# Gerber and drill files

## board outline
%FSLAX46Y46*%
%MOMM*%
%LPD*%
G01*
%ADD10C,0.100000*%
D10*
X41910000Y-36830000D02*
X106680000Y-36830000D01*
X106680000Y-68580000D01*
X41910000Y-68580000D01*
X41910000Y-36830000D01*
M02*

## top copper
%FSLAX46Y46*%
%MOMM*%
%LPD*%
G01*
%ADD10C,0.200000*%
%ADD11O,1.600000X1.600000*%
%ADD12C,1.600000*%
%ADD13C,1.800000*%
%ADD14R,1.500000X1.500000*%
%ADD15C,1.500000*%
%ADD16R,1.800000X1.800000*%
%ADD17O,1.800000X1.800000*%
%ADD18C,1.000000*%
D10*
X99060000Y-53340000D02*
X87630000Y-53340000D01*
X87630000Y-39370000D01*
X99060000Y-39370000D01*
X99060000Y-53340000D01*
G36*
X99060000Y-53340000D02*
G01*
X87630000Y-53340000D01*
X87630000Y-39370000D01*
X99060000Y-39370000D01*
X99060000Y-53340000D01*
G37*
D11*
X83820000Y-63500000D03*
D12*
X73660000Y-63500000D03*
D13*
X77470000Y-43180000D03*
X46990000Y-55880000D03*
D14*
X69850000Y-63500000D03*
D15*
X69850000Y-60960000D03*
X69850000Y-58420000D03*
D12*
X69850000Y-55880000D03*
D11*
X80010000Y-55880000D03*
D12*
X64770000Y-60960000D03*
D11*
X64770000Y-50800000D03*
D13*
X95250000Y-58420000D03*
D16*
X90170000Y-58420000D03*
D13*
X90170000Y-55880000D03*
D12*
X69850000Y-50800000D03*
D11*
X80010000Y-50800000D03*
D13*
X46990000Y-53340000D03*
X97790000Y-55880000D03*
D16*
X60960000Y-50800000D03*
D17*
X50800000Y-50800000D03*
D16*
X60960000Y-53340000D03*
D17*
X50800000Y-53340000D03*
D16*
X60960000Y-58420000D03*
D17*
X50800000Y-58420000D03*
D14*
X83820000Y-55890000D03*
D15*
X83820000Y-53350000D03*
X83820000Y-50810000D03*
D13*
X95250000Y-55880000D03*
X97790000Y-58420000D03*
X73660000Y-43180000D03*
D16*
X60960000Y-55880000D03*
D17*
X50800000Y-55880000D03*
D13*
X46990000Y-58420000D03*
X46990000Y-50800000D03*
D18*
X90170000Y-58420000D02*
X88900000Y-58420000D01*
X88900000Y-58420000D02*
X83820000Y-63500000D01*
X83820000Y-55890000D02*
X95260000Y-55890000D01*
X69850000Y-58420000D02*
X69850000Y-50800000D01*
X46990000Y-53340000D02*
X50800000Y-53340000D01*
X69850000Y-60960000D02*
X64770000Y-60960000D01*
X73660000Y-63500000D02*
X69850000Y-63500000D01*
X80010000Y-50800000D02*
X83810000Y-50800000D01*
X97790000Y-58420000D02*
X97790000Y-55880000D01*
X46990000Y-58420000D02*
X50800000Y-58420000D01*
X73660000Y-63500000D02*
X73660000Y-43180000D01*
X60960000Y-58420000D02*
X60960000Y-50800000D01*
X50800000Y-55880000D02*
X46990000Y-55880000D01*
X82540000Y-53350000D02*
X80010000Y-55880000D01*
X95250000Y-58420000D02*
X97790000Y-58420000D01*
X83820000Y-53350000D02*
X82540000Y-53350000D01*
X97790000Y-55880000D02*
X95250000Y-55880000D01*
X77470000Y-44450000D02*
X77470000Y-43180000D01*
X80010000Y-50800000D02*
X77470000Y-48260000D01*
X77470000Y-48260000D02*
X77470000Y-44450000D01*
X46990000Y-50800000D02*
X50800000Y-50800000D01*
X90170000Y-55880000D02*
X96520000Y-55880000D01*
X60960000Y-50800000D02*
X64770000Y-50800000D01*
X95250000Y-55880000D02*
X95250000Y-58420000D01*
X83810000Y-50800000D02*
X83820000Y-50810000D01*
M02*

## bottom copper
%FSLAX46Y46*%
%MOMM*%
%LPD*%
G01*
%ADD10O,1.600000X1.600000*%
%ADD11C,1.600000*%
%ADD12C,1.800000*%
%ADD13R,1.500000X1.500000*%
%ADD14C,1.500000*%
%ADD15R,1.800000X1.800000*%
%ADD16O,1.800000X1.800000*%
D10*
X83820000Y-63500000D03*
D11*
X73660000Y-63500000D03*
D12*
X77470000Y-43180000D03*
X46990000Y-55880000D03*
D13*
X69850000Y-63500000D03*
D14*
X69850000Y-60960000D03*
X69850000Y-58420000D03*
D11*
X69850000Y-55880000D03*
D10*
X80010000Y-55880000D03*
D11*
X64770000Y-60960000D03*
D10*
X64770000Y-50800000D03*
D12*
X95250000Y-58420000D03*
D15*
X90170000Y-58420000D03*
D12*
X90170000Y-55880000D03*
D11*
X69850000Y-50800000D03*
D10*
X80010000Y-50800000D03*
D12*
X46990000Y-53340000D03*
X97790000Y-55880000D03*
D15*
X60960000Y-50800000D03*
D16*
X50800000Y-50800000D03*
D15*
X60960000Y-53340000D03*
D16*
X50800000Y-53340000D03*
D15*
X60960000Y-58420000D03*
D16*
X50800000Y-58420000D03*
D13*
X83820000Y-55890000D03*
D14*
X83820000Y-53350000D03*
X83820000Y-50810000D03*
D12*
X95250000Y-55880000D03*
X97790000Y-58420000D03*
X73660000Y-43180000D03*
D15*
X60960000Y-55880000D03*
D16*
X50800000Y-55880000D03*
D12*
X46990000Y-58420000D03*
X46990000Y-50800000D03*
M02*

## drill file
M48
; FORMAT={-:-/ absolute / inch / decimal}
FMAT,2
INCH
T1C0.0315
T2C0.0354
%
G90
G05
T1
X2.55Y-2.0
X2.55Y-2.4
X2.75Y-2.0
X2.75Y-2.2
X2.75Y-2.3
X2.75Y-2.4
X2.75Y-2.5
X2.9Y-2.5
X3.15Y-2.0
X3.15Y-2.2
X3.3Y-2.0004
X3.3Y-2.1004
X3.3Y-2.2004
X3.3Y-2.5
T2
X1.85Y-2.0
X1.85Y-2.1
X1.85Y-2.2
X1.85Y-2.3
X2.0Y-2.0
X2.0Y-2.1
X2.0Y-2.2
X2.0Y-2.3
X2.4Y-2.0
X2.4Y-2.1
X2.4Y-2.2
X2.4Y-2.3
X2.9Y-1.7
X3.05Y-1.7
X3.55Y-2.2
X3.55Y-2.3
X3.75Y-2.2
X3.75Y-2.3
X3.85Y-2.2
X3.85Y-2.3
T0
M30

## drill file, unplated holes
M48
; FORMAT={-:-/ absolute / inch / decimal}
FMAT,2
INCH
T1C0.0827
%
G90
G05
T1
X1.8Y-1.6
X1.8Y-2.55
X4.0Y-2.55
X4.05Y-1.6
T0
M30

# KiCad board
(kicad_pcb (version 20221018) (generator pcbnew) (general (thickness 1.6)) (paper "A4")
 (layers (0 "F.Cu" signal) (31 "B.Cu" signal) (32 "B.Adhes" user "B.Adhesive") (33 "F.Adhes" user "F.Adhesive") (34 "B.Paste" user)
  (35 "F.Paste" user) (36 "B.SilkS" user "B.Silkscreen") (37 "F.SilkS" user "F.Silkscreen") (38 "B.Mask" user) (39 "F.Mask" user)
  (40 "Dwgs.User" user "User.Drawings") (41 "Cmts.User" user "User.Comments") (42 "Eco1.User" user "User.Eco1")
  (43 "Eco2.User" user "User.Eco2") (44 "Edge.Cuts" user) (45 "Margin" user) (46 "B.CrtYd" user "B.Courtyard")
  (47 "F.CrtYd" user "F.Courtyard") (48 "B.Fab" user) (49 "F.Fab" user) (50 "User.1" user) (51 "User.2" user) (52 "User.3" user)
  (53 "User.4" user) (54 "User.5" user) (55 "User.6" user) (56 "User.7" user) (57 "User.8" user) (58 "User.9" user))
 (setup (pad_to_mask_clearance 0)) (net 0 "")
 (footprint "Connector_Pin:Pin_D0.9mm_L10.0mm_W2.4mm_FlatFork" (layer "F.Cu") (at 77.47 43.18)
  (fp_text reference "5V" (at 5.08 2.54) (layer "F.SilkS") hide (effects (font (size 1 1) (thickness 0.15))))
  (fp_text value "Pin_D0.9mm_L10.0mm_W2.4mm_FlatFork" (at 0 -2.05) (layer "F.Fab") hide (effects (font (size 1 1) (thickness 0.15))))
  (pad "1" thru_hole circle (at 0 0) (size 1.8 1.8) (drill 0.9) (layers "*.Cu" "*.Mask")))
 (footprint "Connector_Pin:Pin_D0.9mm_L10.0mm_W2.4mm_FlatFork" (layer "F.Cu") (at 46.99 55.88)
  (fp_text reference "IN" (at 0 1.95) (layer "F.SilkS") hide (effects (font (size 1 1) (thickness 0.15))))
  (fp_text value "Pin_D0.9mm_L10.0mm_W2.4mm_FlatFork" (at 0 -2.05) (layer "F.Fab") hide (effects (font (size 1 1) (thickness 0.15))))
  (pad "1" thru_hole circle (at 0 0) (size 1.8 1.8) (drill 0.9) (layers "*.Cu" "*.Mask")))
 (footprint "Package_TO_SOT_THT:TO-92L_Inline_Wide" (layer "F.Cu") (at 69.85 63.5 90)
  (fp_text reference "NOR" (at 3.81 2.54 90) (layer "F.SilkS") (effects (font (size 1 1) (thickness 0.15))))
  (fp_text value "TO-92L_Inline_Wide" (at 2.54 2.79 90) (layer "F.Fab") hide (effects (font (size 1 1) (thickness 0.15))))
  (pad "1" thru_hole rect (at 0 0 90) (size 1.5 1.5) (drill 0.8) (layers "*.Cu" "*.Mask"))
  (pad "2" thru_hole circle (at 2.54 0 90) (size 1.5 1.5) (drill 0.8) (layers "*.Cu" "*.Mask"))
  (pad "3" thru_hole circle (at 5.08 0 90) (size 1.5 1.5) (drill 0.8) (layers "*.Cu" "*.Mask")))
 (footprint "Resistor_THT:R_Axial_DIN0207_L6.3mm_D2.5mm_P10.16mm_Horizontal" (layer "F.Cu") (at 69.85 55.88)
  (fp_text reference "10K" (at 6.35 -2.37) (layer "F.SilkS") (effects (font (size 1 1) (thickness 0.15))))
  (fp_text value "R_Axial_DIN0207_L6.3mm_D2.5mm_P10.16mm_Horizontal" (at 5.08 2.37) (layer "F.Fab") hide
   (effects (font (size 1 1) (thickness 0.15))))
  (pad "1" thru_hole circle (at 0 0) (size 1.6 1.6) (drill 0.8) (layers "*.Cu" "*.Mask"))
  (pad "2" thru_hole oval (at 10.16 0) (size 1.6 1.6) (drill 0.8) (layers "*.Cu" "*.Mask")))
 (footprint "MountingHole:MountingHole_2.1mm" (layer "F.Cu") (at 101.6 64.77)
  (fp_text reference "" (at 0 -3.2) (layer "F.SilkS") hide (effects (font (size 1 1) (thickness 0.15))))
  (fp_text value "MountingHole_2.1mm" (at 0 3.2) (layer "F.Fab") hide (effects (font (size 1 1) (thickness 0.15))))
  (pad "" np_thru_hole circle (at 0 0) (size 2.1 2.1) (drill 2.1) (layers "F&B.Cu" "*.Mask")))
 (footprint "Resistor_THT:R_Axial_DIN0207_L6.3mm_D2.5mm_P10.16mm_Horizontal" (layer "F.Cu") (at 64.77 60.96 90)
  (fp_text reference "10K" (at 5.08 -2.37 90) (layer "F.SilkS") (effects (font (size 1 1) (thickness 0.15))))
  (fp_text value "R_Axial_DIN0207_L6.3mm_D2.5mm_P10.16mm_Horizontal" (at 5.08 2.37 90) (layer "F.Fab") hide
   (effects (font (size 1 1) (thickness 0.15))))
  (pad "1" thru_hole circle (at 0 0 90) (size 1.6 1.6) (drill 0.8) (layers "*.Cu" "*.Mask"))
  (pad "2" thru_hole oval (at 10.16 0 90) (size 1.6 1.6) (drill 0.8) (layers "*.Cu" "*.Mask")))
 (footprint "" (layer "F.Cu") (at 95.25 58.42)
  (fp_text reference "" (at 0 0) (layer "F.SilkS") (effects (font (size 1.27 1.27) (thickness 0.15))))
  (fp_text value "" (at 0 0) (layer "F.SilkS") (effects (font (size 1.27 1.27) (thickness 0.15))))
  (pad "1" thru_hole circle (at 0 0) (size 1.8 1.8) (drill 0.9) (layers "*.Cu" "*.Mask")))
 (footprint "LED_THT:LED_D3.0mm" (layer "F.Cu") (at 90.17 58.42 90)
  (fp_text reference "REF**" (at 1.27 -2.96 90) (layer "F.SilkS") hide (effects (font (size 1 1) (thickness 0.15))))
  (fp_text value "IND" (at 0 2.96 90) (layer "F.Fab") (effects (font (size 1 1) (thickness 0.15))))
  (pad "1" thru_hole rect (at 0 0 90) (size 1.8 1.8) (drill 0.9) (layers "*.Cu" "*.Mask"))
  (pad "2" thru_hole circle (at 2.54 0 90) (size 1.8 1.8) (drill 0.9) (layers "*.Cu" "*.Mask")))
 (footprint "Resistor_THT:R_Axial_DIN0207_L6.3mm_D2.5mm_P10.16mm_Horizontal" (layer "F.Cu") (at 69.85 50.8)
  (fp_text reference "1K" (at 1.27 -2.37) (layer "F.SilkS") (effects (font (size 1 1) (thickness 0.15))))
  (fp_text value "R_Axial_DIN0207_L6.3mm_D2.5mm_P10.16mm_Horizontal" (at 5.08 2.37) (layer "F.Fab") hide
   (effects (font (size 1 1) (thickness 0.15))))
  (pad "1" thru_hole circle (at 0 0) (size 1.6 1.6) (drill 0.8) (layers "*.Cu" "*.Mask"))
  (pad "2" thru_hole oval (at 10.16 0) (size 1.6 1.6) (drill 0.8) (layers "*.Cu" "*.Mask")))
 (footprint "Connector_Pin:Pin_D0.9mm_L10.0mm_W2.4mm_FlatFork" (layer "F.Cu") (at 46.99 53.34)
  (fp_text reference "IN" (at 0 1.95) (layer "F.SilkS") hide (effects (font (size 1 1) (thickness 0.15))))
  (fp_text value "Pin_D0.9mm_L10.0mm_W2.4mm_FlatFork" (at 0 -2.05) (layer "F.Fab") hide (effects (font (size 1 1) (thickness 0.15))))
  (pad "1" thru_hole circle (at 0 0) (size 1.8 1.8) (drill 0.9) (layers "*.Cu" "*.Mask")))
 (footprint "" (layer "F.Cu") (at 97.79 55.88)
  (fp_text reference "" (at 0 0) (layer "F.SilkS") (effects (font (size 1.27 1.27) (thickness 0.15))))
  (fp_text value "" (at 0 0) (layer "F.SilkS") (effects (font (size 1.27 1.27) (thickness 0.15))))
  (pad "1" thru_hole circle (at 0 0) (size 1.8 1.8) (drill 0.9) (layers "*.Cu" "*.Mask")))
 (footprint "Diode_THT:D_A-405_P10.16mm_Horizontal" (layer "F.Cu") (at 60.96 50.8 180)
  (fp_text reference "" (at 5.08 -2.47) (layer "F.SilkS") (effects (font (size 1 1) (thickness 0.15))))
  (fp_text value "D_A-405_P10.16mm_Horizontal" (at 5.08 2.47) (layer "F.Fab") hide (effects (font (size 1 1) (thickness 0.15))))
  (pad "1" thru_hole rect (at 0 0 180) (size 1.8 1.8) (drill 0.9) (layers "*.Cu" "*.Mask"))
  (pad "2" thru_hole oval (at 10.16 0 180) (size 1.8 1.8) (drill 0.9) (layers "*.Cu" "*.Mask")))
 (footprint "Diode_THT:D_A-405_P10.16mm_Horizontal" (layer "F.Cu") (at 60.96 53.34 180)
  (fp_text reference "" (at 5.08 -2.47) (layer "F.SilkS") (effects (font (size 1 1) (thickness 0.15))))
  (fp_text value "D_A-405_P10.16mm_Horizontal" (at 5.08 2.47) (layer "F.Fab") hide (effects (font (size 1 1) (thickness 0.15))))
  (pad "1" thru_hole rect (at 0 0 180) (size 1.8 1.8) (drill 0.9) (layers "*.Cu" "*.Mask"))
  (pad "2" thru_hole oval (at 10.16 0 180) (size 1.8 1.8) (drill 0.9) (layers "*.Cu" "*.Mask")))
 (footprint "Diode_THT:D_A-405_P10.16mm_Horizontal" (layer "F.Cu") (at 60.96 58.42 180)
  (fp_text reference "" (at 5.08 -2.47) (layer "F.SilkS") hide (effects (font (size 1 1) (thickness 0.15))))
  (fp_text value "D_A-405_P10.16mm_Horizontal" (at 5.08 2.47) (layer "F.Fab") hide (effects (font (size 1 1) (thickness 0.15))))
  (pad "1" thru_hole rect (at 0 0 180) (size 1.8 1.8) (drill 0.9) (layers "*.Cu" "*.Mask"))
  (pad "2" thru_hole oval (at 10.16 0 180) (size 1.8 1.8) (drill 0.9) (layers "*.Cu" "*.Mask")))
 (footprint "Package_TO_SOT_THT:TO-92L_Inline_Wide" (layer "F.Cu") (at 83.82 55.89 90)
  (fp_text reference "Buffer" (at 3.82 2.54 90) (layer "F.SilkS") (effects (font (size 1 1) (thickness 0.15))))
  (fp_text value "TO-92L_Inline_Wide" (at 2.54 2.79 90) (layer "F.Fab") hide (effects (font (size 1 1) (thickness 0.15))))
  (pad "1" thru_hole rect (at 0 0 90) (size 1.5 1.5) (drill 0.8) (layers "*.Cu" "*.Mask"))
  (pad "2" thru_hole circle (at 2.54 0 90) (size 1.5 1.5) (drill 0.8) (layers "*.Cu" "*.Mask"))
  (pad "3" thru_hole circle (at 5.08 0 90) (size 1.5 1.5) (drill 0.8) (layers "*.Cu" "*.Mask")))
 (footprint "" (layer "F.Cu") (at 95.25 55.88)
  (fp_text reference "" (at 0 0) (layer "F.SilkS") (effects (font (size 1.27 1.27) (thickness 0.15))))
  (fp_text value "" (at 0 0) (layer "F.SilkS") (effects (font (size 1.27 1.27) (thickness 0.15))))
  (pad "1" thru_hole circle (at 0 0) (size 1.8 1.8) (drill 0.9) (layers "*.Cu" "*.Mask")))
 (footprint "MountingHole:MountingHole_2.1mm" (layer "F.Cu") (at 45.72 64.77)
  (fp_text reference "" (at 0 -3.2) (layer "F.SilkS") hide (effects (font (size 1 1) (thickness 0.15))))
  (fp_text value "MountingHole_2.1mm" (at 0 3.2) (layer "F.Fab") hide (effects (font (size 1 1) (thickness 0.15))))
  (pad "" np_thru_hole circle (at 0 0) (size 2.1 2.1) (drill 2.1) (layers "F&B.Cu" "*.Mask")))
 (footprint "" (layer "F.Cu") (at 97.79 58.42)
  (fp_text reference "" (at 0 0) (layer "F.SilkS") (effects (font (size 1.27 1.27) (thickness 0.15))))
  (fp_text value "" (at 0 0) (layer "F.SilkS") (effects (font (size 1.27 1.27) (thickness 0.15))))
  (pad "1" thru_hole circle (at 0 0) (size 1.8 1.8) (drill 0.9) (layers "*.Cu" "*.Mask")))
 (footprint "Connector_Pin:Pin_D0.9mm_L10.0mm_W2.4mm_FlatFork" (layer "F.Cu") (at 73.66 43.18)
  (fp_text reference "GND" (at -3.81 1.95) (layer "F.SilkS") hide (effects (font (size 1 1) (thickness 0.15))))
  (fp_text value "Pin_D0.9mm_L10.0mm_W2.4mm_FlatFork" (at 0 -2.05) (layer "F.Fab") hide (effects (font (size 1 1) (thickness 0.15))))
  (pad "1" thru_hole circle (at 0 0) (size 1.8 1.8) (drill 0.9) (layers "*.Cu" "*.Mask")))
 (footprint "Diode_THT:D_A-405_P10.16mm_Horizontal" (layer "F.Cu") (at 60.96 55.88 180)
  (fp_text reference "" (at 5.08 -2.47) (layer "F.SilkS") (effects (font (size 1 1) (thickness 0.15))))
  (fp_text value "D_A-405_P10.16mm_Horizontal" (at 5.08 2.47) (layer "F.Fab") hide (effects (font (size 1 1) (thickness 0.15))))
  (pad "1" thru_hole rect (at 0 0 180) (size 1.8 1.8) (drill 0.9) (layers "*.Cu" "*.Mask"))
  (pad "2" thru_hole oval (at 10.16 0 180) (size 1.8 1.8) (drill 0.9) (layers "*.Cu" "*.Mask")))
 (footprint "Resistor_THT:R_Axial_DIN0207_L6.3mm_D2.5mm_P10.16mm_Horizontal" (layer "F.Cu") (at 73.66 63.5)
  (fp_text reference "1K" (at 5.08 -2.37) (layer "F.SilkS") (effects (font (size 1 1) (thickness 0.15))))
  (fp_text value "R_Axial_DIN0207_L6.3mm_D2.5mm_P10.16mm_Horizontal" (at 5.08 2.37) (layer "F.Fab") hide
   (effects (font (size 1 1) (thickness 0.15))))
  (pad "1" thru_hole circle (at 0 0) (size 1.6 1.6) (drill 0.8) (layers "*.Cu" "*.Mask"))
  (pad "2" thru_hole oval (at 10.16 0) (size 1.6 1.6) (drill 0.8) (layers "*.Cu" "*.Mask")))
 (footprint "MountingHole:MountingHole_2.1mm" (layer "F.Cu") (at 45.72 40.64)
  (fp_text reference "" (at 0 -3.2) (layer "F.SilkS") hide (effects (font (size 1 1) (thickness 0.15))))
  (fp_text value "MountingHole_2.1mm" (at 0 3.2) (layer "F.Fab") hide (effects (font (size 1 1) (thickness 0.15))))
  (pad "" np_thru_hole circle (at 0 0) (size 2.1 2.1) (drill 2.1) (layers "F&B.Cu" "*.Mask")))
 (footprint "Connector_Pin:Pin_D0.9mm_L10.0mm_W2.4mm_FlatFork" (layer "F.Cu") (at 46.99 58.42)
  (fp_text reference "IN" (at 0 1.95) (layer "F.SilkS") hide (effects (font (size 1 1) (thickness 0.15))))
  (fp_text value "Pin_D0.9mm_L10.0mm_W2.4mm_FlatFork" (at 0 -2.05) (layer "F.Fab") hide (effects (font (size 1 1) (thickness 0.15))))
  (pad "1" thru_hole circle (at 0 0) (size 1.8 1.8) (drill 0.9) (layers "*.Cu" "*.Mask")))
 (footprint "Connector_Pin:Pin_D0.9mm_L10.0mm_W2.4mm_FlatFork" (layer "F.Cu") (at 46.99 50.8)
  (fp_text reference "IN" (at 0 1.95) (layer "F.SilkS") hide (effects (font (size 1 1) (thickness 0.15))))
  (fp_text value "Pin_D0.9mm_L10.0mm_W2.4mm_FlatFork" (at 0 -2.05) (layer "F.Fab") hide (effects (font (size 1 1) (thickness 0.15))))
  (pad "1" thru_hole circle (at 0 0) (size 1.8 1.8) (drill 0.9) (layers "*.Cu" "*.Mask")))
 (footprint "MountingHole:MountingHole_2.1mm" (layer "F.Cu") (at 102.87 40.64)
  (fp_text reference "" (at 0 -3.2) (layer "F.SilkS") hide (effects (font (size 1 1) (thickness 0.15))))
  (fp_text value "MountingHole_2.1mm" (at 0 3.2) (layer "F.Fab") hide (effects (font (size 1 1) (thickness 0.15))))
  (pad "" np_thru_hole circle (at 0 0) (size 2.1 2.1) (drill 2.1) (layers "F&B.Cu" "*.Mask")))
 (gr_poly
  (pts (xy 99.06 39.37) (xy 99.06 53.34) (xy 87.63 53.34) (xy 87.63 39.37)) (stroke (width 0.2) (type solid)) (fill solid) (layer "F.Cu"))
 (gr_rect (start 41.91 36.83) (end 106.68 68.58) (stroke (width 0.1) (type default)) (fill none) (layer "Edge.Cuts"))
 (segment (start 69.85 58.42) (end 69.85 50.8) (width 1) (layer "F.Cu") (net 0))
 (segment (start 46.99 53.34) (end 50.8 53.34) (width 1) (layer "F.Cu") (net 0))
 (segment (start 69.85 60.96) (end 64.77 60.96) (width 1) (layer "F.Cu") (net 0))
 (segment (start 73.66 63.5) (end 69.85 63.5) (width 1) (layer "F.Cu") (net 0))
 (segment (start 80.01 50.8) (end 83.81 50.8) (width 1) (layer "F.Cu") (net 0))
 (segment (start 97.79 58.42) (end 97.79 55.88) (width 1) (layer "F.Cu") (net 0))
 (segment (start 46.99 58.42) (end 50.8 58.42) (width 1) (layer "F.Cu") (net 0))
 (segment (start 73.66 63.5) (end 73.66 43.18) (width 1) (layer "F.Cu") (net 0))
 (segment (start 60.96 58.42) (end 60.96 50.8) (width 1) (layer "F.Cu") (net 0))
 (segment (start 50.8 55.88) (end 46.99 55.88) (width 1) (layer "F.Cu") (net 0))
 (segment (start 82.54 53.35) (end 80.01 55.88) (width 1) (layer "F.Cu") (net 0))
 (segment (start 95.25 58.42) (end 97.79 58.42) (width 1) (layer "F.Cu") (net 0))
 (segment (start 83.82 53.35) (end 82.54 53.35) (width 1) (layer "F.Cu") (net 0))
 (segment (start 97.79 55.88) (end 95.25 55.88) (width 1) (layer "F.Cu") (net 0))
 (segment (start 77.47 44.45) (end 77.47 43.18) (width 1) (layer "F.Cu") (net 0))
 (segment (start 80.01 50.8) (end 77.47 48.26) (width 1) (layer "F.Cu") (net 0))
 (segment (start 77.47 48.26) (end 77.47 44.45) (width 1) (layer "F.Cu") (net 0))
 (segment (start 46.99 50.8) (end 50.8 50.8) (width 1) (layer "F.Cu") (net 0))
 (segment (start 90.17 58.42) (end 88.9 58.42) (width 1) (layer "F.Cu") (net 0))
 (segment (start 90.17 55.88) (end 96.52 55.88) (width 1) (layer "F.Cu") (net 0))
 (segment (start 60.96 50.8) (end 64.77 50.8) (width 1) (layer "F.Cu") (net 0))
 (segment (start 83.82 55.89) (end 95.26 55.89) (width 1) (layer "F.Cu") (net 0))
 (segment (start 88.9 58.42) (end 83.82 63.5) (width 1) (layer "F.Cu") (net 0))
 (segment (start 95.25 55.88) (end 95.25 58.42) (width 1) (layer "F.Cu") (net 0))
 (segment (start 83.81 50.8) (end 83.82 50.81) (width 1) (layer "F.Cu") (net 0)))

